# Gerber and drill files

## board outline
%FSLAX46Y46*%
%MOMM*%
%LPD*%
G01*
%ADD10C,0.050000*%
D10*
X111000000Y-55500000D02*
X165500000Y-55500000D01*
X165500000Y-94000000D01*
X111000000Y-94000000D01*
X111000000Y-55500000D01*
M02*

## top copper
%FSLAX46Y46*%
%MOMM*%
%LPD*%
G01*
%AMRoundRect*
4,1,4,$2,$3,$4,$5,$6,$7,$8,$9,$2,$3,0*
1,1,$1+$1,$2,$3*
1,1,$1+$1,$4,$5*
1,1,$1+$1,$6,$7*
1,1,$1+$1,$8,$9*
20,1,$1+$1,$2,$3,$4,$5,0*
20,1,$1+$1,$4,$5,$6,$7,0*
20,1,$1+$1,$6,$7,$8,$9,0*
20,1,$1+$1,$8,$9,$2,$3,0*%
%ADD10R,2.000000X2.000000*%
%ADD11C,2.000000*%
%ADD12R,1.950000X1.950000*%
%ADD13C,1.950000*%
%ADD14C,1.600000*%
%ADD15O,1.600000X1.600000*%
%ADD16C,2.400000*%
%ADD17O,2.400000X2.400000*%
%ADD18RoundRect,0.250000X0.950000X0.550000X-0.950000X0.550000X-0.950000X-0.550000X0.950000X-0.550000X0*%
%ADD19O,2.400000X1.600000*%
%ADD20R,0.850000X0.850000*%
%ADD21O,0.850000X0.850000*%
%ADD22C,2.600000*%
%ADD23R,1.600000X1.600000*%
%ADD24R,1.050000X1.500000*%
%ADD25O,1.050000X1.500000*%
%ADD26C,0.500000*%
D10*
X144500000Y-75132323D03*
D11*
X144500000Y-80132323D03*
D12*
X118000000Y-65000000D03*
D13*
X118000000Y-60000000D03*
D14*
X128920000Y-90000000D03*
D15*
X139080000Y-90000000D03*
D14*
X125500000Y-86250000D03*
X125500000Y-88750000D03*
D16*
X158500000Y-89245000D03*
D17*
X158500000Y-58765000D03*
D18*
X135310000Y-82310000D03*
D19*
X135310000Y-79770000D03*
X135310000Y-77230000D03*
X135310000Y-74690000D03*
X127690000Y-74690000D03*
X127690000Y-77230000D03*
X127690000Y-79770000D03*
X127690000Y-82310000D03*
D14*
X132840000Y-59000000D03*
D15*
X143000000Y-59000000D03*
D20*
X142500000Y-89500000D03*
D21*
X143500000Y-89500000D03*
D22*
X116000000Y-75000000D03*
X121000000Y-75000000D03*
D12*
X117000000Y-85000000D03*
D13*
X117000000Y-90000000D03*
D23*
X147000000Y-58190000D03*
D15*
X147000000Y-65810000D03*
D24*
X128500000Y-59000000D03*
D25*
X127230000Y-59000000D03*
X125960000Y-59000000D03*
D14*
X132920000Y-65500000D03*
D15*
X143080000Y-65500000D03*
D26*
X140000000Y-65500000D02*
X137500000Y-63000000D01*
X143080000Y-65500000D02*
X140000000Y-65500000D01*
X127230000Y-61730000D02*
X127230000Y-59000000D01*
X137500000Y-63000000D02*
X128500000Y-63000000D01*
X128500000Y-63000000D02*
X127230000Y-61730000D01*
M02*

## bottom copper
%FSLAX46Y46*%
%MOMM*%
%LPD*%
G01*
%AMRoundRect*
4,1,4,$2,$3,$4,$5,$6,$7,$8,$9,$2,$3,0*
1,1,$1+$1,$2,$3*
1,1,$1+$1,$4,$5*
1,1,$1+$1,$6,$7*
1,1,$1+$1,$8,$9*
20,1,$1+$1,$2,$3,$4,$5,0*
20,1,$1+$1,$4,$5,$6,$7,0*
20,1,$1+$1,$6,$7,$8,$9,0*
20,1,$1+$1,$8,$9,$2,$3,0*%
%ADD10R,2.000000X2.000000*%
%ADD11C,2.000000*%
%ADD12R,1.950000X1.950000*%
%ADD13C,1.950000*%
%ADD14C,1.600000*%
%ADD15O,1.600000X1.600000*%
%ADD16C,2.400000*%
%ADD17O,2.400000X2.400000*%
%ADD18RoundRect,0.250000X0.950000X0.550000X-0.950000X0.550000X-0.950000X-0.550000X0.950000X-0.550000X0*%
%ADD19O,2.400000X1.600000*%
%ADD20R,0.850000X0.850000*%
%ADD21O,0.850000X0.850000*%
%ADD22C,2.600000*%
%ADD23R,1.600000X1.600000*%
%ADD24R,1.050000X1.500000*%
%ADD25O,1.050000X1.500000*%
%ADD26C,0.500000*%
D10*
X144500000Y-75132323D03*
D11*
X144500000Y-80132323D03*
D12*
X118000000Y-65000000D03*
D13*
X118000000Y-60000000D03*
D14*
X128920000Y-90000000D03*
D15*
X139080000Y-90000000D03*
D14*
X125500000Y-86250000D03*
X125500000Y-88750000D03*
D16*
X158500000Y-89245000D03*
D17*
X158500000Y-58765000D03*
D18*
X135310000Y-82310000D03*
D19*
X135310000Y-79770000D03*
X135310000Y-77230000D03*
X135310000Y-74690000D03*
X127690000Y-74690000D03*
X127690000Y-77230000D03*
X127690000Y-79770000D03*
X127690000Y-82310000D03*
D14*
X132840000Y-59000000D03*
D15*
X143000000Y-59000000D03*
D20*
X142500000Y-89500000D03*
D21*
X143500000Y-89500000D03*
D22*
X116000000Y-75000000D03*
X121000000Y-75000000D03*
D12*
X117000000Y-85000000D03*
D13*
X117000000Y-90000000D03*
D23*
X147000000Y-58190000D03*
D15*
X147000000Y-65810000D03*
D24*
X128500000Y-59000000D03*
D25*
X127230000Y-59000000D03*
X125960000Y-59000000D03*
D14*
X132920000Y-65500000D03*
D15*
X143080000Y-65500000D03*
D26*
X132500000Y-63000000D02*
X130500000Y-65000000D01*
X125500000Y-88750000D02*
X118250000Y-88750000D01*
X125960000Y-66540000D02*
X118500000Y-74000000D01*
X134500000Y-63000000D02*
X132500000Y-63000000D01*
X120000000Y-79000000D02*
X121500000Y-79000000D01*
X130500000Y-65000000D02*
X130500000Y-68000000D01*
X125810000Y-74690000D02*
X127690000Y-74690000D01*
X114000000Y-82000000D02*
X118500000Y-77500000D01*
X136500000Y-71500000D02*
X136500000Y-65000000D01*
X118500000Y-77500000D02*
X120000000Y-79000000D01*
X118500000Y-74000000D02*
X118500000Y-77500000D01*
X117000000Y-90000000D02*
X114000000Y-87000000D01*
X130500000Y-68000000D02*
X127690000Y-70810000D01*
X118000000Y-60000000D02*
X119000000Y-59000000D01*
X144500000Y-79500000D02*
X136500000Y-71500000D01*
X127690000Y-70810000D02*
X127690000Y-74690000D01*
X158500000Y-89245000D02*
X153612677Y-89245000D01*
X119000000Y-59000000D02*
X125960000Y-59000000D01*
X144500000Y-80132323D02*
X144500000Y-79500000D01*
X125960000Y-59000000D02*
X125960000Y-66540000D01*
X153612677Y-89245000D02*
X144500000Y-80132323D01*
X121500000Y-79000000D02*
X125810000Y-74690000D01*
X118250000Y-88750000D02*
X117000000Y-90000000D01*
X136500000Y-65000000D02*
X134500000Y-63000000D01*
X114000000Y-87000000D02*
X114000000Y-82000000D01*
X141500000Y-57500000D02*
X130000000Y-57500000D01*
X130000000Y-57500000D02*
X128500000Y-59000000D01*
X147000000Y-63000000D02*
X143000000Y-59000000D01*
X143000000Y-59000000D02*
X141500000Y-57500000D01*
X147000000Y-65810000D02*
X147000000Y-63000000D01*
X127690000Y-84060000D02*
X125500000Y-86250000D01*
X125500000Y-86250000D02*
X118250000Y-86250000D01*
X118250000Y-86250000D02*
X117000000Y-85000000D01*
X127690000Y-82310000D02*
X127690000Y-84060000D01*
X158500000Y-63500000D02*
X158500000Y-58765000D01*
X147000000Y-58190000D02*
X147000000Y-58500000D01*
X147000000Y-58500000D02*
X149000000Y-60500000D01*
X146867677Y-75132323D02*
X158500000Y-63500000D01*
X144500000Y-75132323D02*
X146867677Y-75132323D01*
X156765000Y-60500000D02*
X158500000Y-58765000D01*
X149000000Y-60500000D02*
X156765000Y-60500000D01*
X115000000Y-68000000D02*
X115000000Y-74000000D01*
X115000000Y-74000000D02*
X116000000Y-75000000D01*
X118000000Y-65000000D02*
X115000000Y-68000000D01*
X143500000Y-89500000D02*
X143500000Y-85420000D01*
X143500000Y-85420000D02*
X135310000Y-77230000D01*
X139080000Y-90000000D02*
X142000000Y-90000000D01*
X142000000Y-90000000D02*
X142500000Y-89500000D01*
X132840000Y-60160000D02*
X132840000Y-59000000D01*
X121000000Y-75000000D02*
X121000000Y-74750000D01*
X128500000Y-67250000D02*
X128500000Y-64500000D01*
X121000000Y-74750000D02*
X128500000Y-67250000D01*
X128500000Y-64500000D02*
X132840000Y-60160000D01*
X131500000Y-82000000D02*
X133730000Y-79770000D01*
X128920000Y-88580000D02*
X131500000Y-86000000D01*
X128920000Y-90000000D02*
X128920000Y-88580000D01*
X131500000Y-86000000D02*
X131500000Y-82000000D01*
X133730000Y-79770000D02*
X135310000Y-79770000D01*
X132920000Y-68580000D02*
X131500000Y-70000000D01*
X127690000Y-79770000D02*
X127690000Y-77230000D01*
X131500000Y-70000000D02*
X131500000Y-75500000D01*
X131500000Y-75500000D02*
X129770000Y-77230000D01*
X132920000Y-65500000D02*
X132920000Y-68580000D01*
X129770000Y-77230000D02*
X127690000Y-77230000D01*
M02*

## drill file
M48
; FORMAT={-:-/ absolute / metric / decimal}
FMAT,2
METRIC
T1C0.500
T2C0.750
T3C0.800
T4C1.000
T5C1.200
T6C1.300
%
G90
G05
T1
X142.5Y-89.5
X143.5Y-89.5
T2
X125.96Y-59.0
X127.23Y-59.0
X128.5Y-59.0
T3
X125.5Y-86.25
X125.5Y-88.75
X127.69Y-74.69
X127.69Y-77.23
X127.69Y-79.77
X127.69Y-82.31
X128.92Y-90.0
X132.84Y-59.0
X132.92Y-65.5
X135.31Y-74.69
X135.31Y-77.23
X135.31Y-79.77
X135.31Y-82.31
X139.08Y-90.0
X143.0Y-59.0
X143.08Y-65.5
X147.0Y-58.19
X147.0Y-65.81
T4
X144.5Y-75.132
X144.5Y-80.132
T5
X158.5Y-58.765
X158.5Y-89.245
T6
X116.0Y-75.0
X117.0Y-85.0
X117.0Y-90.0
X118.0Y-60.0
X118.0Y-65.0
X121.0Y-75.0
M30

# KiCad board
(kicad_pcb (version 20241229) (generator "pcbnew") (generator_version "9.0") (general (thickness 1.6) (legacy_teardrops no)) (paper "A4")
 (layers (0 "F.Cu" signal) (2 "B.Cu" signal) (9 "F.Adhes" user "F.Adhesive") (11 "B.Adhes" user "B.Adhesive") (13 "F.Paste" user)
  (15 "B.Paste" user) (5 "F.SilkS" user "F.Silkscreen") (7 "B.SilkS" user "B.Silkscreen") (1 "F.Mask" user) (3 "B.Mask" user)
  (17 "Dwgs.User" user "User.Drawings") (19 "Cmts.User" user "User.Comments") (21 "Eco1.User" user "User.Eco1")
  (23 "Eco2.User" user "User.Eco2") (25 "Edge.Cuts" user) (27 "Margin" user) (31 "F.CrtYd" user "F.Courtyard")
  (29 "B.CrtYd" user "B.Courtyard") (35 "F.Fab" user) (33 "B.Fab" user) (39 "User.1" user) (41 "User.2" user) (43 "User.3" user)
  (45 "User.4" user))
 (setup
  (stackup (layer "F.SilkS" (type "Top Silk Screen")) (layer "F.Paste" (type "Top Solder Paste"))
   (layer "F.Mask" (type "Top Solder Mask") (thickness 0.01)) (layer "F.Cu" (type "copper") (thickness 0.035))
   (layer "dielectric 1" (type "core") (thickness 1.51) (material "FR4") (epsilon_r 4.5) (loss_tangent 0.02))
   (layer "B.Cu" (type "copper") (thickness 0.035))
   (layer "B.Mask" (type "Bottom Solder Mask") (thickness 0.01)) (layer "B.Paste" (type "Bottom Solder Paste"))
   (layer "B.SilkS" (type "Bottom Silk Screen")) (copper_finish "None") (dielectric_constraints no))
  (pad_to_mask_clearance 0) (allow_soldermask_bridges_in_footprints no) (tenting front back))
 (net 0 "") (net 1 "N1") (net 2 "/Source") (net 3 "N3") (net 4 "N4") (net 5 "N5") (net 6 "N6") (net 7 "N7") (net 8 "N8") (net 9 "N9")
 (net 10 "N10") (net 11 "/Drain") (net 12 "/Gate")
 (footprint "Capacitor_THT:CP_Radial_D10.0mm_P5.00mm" (layer "F.Cu") (at 144.5 75.132323 -90)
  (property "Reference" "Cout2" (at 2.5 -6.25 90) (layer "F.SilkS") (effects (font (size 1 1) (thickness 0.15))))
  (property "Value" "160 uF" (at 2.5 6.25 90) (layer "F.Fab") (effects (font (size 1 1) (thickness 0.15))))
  (pad "1" thru_hole rect (at 0 0 270) (size 2 2) (drill 1) (layers "*.Cu" "*.Mask") (remove_unused_layers no) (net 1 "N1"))
  (pad "2" thru_hole circle (at 5 0 270) (size 2 2) (drill 1) (layers "*.Cu" "*.Mask") (remove_unused_layers no) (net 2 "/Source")))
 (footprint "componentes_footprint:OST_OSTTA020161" (layer "F.Cu") (at 118 62.5 90)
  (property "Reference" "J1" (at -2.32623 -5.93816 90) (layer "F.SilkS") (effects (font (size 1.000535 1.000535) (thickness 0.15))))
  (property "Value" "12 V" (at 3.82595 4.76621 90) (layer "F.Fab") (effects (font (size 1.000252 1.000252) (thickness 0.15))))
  (pad "1" thru_hole rect (at -2.5 0 90) (size 1.95 1.95) (drill 1.3) (layers "*.Cu" "*.Mask") (remove_unused_layers no) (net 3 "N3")
   (solder_mask_margin 0.102))
  (pad "2" thru_hole circle (at 2.5 0 90) (size 1.95 1.95) (drill 1.3) (layers "*.Cu" "*.Mask") (remove_unused_layers no) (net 2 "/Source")
   (solder_mask_margin 0.102)))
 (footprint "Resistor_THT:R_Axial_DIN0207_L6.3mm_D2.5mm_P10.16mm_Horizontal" (layer "F.Cu") (at 128.92 90)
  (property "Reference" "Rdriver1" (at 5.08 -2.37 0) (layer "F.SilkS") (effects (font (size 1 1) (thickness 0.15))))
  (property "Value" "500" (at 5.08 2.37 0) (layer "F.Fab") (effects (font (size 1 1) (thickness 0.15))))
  (pad "1" thru_hole circle (at 0 0) (size 1.6 1.6) (drill 0.8) (layers "*.Cu" "*.Mask") (remove_unused_layers no) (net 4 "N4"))
  (pad "2" thru_hole oval (at 10.16 0) (size 1.6 1.6) (drill 0.8) (layers "*.Cu" "*.Mask") (remove_unused_layers no) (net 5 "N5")))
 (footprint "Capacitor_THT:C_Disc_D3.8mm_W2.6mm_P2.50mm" (layer "F.Cu") (at 125.5 86.25 -90)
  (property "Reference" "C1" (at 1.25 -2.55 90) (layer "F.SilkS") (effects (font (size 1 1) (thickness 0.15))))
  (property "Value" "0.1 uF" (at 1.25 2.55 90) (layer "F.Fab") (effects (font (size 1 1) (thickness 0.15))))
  (pad "1" thru_hole circle (at 0 0 270) (size 1.6 1.6) (drill 0.8) (layers "*.Cu" "*.Mask") (remove_unused_layers no) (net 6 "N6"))
  (pad "2" thru_hole circle (at 2.5 0 270) (size 1.6 1.6) (drill 0.8) (layers "*.Cu" "*.Mask") (remove_unused_layers no) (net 2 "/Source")))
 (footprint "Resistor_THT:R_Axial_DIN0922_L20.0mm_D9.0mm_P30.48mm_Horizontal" (layer "F.Cu") (at 158.5 89.245 90)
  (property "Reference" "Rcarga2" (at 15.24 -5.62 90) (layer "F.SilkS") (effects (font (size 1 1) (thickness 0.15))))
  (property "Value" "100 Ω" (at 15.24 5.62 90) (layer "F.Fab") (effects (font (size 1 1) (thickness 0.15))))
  (pad "1" thru_hole circle (at 0 0 90) (size 2.4 2.4) (drill 1.2) (layers "*.Cu" "*.Mask") (remove_unused_layers no) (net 2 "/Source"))
  (pad "2" thru_hole oval (at 30.48 0 90) (size 2.4 2.4) (drill 1.2) (layers "*.Cu" "*.Mask") (remove_unused_layers no) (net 1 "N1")))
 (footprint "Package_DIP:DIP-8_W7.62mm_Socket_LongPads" (layer "F.Cu") (at 135.31 82.31 180)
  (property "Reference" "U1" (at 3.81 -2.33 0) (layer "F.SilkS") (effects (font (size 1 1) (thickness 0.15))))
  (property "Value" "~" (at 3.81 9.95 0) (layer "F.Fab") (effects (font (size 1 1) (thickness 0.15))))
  (pad "1" thru_hole roundrect (at 0 0 180) (size 2.4 1.6) (drill 0.8) (layers "*.Cu" "*.Mask") (remove_unused_layers no)
   (roundrect_rratio 0.15625) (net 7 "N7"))
  (pad "2" thru_hole oval (at 0 2.54 180) (size 2.4 1.6) (drill 0.8) (layers "*.Cu" "*.Mask") (remove_unused_layers no) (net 4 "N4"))
  (pad "3" thru_hole oval (at 0 5.08 180) (size 2.4 1.6) (drill 0.8) (layers "*.Cu" "*.Mask") (remove_unused_layers no) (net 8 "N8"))
  (pad "4" thru_hole oval (at 0 7.62 180) (size 2.4 1.6) (drill 0.8) (layers "*.Cu" "*.Mask") (remove_unused_layers no))
  (pad "5" thru_hole oval (at 7.62 7.62 180) (size 2.4 1.6) (drill 0.8) (layers "*.Cu" "*.Mask") (remove_unused_layers no) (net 2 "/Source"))
  (pad "6" thru_hole oval (at 7.62 5.08 180) (size 2.4 1.6) (drill 0.8) (layers "*.Cu" "*.Mask") (remove_unused_layers no) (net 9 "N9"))
  (pad "7" thru_hole oval (at 7.62 2.54 180) (size 2.4 1.6) (drill 0.8) (layers "*.Cu" "*.Mask") (remove_unused_layers no) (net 9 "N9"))
  (pad "8" thru_hole oval (at 7.62 0 180) (size 2.4 1.6) (drill 0.8) (layers "*.Cu" "*.Mask") (remove_unused_layers no) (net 6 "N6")))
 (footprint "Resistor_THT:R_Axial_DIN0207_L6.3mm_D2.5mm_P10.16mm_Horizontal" (layer "F.Cu") (at 132.84 59)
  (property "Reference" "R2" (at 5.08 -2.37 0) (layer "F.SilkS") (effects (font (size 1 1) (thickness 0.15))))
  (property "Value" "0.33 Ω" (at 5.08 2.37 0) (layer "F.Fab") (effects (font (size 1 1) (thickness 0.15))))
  (pad "1" thru_hole circle (at 0 0) (size 1.6 1.6) (drill 0.8) (layers "*.Cu" "*.Mask") (remove_unused_layers no) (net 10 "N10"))
  (pad "2" thru_hole oval (at 10.16 0) (size 1.6 1.6) (drill 0.8) (layers "*.Cu" "*.Mask") (remove_unused_layers no) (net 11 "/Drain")))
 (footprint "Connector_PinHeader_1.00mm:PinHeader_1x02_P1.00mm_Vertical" (layer "F.Cu") (at 142.5 89.5 90)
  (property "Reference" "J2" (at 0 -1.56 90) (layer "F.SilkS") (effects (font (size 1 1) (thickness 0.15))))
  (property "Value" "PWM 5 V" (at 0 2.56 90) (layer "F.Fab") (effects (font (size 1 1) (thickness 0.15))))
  (pad "1" thru_hole rect (at 0 0 90) (size 0.85 0.85) (drill 0.5) (layers "*.Cu" "*.Mask") (remove_unused_layers no) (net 5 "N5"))
  (pad "2" thru_hole oval (at 0 1 90) (size 0.85 0.85) (drill 0.5) (layers "*.Cu" "*.Mask") (remove_unused_layers no) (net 8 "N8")))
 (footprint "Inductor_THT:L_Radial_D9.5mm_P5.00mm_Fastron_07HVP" (layer "F.Cu") (at 116 75)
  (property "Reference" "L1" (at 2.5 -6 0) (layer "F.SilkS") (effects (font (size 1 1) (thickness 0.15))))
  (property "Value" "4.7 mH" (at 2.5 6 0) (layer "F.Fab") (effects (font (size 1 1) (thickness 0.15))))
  (pad "1" thru_hole circle (at 0 0) (size 2.6 2.6) (drill 1.3) (layers "*.Cu" "*.Mask") (remove_unused_layers no) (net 3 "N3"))
  (pad "2" thru_hole circle (at 5 0) (size 2.6 2.6) (drill 1.3) (layers "*.Cu" "*.Mask") (remove_unused_layers no) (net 10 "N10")))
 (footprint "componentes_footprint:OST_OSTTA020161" (layer "F.Cu") (at 117 87.5 -90)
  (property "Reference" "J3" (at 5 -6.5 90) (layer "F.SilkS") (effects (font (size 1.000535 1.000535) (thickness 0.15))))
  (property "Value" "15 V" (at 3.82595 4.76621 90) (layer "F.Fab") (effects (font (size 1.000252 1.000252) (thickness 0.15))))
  (pad "1" thru_hole rect (at -2.5 0 270) (size 1.95 1.95) (drill 1.3) (layers "*.Cu" "*.Mask") (remove_unused_layers no) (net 6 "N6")
   (solder_mask_margin 0.102))
  (pad "2" thru_hole circle (at 2.5 0 270) (size 1.95 1.95) (drill 1.3) (layers "*.Cu" "*.Mask") (remove_unused_layers no) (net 2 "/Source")
   (solder_mask_margin 0.102)))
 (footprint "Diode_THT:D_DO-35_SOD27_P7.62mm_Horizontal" (layer "F.Cu") (at 147 58.19 -90)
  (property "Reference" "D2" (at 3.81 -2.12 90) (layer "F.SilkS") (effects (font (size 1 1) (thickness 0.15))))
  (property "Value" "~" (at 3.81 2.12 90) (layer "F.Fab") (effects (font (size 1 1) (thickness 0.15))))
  (pad "1" thru_hole rect (at 0 0 270) (size 1.6 1.6) (drill 0.8) (layers "*.Cu" "*.Mask") (remove_unused_layers no) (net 1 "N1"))
  (pad "2" thru_hole oval (at 7.62 0 270) (size 1.6 1.6) (drill 0.8) (layers "*.Cu" "*.Mask") (remove_unused_layers no) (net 11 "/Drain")))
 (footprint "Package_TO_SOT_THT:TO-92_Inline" (layer "F.Cu") (at 128.5 59 180)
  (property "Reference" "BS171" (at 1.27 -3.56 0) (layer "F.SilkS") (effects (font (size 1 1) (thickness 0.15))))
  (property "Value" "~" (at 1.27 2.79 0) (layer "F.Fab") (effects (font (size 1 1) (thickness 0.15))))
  (pad "1" thru_hole rect (at 0 0 180) (size 1.05 1.5) (drill 0.75) (layers "*.Cu" "*.Mask") (remove_unused_layers no) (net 11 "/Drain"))
  (pad "2" thru_hole oval (at 1.27 0 180) (size 1.05 1.5) (drill 0.75) (layers "*.Cu" "*.Mask") (remove_unused_layers no) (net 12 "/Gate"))
  (pad "3" thru_hole oval (at 2.54 0 180) (size 1.05 1.5) (drill 0.75) (layers "*.Cu" "*.Mask") (remove_unused_layers no) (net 2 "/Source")))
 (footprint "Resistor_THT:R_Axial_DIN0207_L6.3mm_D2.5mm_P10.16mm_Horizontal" (layer "F.Cu") (at 132.92 65.5)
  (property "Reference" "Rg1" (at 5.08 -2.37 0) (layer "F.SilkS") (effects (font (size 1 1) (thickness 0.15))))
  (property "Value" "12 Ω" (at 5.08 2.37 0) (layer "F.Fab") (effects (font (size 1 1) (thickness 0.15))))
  (pad "1" thru_hole circle (at 0 0) (size 1.6 1.6) (drill 0.8) (layers "*.Cu" "*.Mask") (remove_unused_layers no) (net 9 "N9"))
  (pad "2" thru_hole oval (at 10.16 0) (size 1.6 1.6) (drill 0.8) (layers "*.Cu" "*.Mask") (remove_unused_layers no) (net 12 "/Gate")))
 (gr_rect (start 111 55.5) (end 165.5 94) (stroke (width 0.05) (type default)) (fill no) (layer "Edge.Cuts"))
 (segment (start 132.5 63) (end 130.5 65) (width 0.5) (layer "B.Cu") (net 2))
 (segment (start 125.5 88.75) (end 118.25 88.75) (width 0.5) (layer "B.Cu") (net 2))
 (segment (start 125.96 66.54) (end 118.5 74) (width 0.5) (layer "B.Cu") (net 2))
 (segment (start 134.5 63) (end 132.5 63) (width 0.5) (layer "B.Cu") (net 2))
 (segment (start 120 79) (end 121.5 79) (width 0.5) (layer "B.Cu") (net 2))
 (segment (start 130.5 65) (end 130.5 68) (width 0.5) (layer "B.Cu") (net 2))
 (segment (start 125.81 74.69) (end 127.69 74.69) (width 0.5) (layer "B.Cu") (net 2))
 (segment (start 114 82) (end 118.5 77.5) (width 0.5) (layer "B.Cu") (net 2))
 (segment (start 136.5 71.5) (end 136.5 65) (width 0.5) (layer "B.Cu") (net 2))
 (segment (start 118.5 77.5) (end 120 79) (width 0.5) (layer "B.Cu") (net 2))
 (segment (start 118.5 74) (end 118.5 77.5) (width 0.5) (layer "B.Cu") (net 2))
 (segment (start 117 90) (end 114 87) (width 0.5) (layer "B.Cu") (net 2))
 (segment (start 130.5 68) (end 127.69 70.81) (width 0.5) (layer "B.Cu") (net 2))
 (segment (start 118 60) (end 119 59) (width 0.5) (layer "B.Cu") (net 2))
 (segment (start 144.5 79.5) (end 136.5 71.5) (width 0.5) (layer "B.Cu") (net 2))
 (segment (start 127.69 70.81) (end 127.69 74.69) (width 0.5) (layer "B.Cu") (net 2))
 (segment (start 158.5 89.245) (end 153.612677 89.245) (width 0.5) (layer "B.Cu") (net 2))
 (segment (start 119 59) (end 125.96 59) (width 0.5) (layer "B.Cu") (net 2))
 (segment (start 144.5 80.132323) (end 144.5 79.5) (width 0.5) (layer "B.Cu") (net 2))
 (segment (start 125.96 59) (end 125.96 66.54) (width 0.5) (layer "B.Cu") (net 2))
 (segment (start 153.612677 89.245) (end 144.5 80.132323) (width 0.5) (layer "B.Cu") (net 2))
 (segment (start 121.5 79) (end 125.81 74.69) (width 0.5) (layer "B.Cu") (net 2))
 (segment (start 118.25 88.75) (end 117 90) (width 0.5) (layer "B.Cu") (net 2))
 (segment (start 136.5 65) (end 134.5 63) (width 0.5) (layer "B.Cu") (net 2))
 (segment (start 114 87) (end 114 82) (width 0.5) (layer "B.Cu") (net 2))
 (segment (start 141.5 57.5) (end 130 57.5) (width 0.5) (layer "B.Cu") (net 11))
 (segment (start 130 57.5) (end 128.5 59) (width 0.5) (layer "B.Cu") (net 11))
 (segment (start 147 63) (end 143 59) (width 0.5) (layer "B.Cu") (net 11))
 (segment (start 143 59) (end 141.5 57.5) (width 0.5) (layer "B.Cu") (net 11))
 (segment (start 147 65.81) (end 147 63) (width 0.5) (layer "B.Cu") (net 11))
 (segment (start 140 65.5) (end 137.5 63) (width 0.5) (layer "F.Cu") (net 12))
 (segment (start 143.08 65.5) (end 140 65.5) (width 0.5) (layer "F.Cu") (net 12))
 (segment (start 127.23 61.73) (end 127.23 59) (width 0.5) (layer "F.Cu") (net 12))
 (segment (start 137.5 63) (end 128.5 63) (width 0.5) (layer "F.Cu") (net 12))
 (segment (start 128.5 63) (end 127.23 61.73) (width 0.5) (layer "F.Cu") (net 12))
 (segment (start 127.69 84.06) (end 125.5 86.25) (width 0.5) (layer "B.Cu") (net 6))
 (segment (start 125.5 86.25) (end 118.25 86.25) (width 0.5) (layer "B.Cu") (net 6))
 (segment (start 118.25 86.25) (end 117 85) (width 0.5) (layer "B.Cu") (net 6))
 (segment (start 127.69 82.31) (end 127.69 84.06) (width 0.5) (layer "B.Cu") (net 6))
 (segment (start 158.5 63.5) (end 158.5 58.765) (width 0.5) (layer "B.Cu") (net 1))
 (segment (start 147 58.19) (end 147 58.5) (width 0.5) (layer "B.Cu") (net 1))
 (segment (start 147 58.5) (end 149 60.5) (width 0.5) (layer "B.Cu") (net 1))
 (segment (start 146.867677 75.132323) (end 158.5 63.5) (width 0.5) (layer "B.Cu") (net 1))
 (segment (start 144.5 75.132323) (end 146.867677 75.132323) (width 0.5) (layer "B.Cu") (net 1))
 (segment (start 156.765 60.5) (end 158.5 58.765) (width 0.5) (layer "B.Cu") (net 1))
 (segment (start 149 60.5) (end 156.765 60.5) (width 0.5) (layer "B.Cu") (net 1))
 (segment (start 115 68) (end 115 74) (width 0.5) (layer "B.Cu") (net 3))
 (segment (start 115 74) (end 116 75) (width 0.5) (layer "B.Cu") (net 3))
 (segment (start 118 65) (end 115 68) (width 0.5) (layer "B.Cu") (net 3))
 (segment (start 143.5 89.5) (end 143.5 85.42) (width 0.5) (layer "B.Cu") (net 8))
 (segment (start 143.5 85.42) (end 135.31 77.23) (width 0.5) (layer "B.Cu") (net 8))
 (segment (start 139.08 90) (end 142 90) (width 0.5) (layer "B.Cu") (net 5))
 (segment (start 142 90) (end 142.5 89.5) (width 0.5) (layer "B.Cu") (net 5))
 (segment (start 132.84 60.16) (end 132.84 59) (width 0.5) (layer "B.Cu") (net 10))
 (segment (start 121 75) (end 121 74.75) (width 0.5) (layer "B.Cu") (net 10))
 (segment (start 128.5 67.25) (end 128.5 64.5) (width 0.5) (layer "B.Cu") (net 10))
 (segment (start 121 74.75) (end 128.5 67.25) (width 0.5) (layer "B.Cu") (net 10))
 (segment (start 128.5 64.5) (end 132.84 60.16) (width 0.5) (layer "B.Cu") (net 10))
 (segment (start 131.5 82) (end 133.73 79.77) (width 0.5) (layer "B.Cu") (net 4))
 (segment (start 128.92 88.58) (end 131.5 86) (width 0.5) (layer "B.Cu") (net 4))
 (segment (start 128.92 90) (end 128.92 88.58) (width 0.5) (layer "B.Cu") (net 4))
 (segment (start 131.5 86) (end 131.5 82) (width 0.5) (layer "B.Cu") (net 4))
 (segment (start 133.73 79.77) (end 135.31 79.77) (width 0.5) (layer "B.Cu") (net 4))
 (segment (start 132.92 68.58) (end 131.5 70) (width 0.5) (layer "B.Cu") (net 9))
 (segment (start 127.69 79.77) (end 127.69 77.23) (width 0.5) (layer "B.Cu") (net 9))
 (segment (start 131.5 70) (end 131.5 75.5) (width 0.5) (layer "B.Cu") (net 9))
 (segment (start 131.5 75.5) (end 129.77 77.23) (width 0.5) (layer "B.Cu") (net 9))
 (segment (start 132.92 65.5) (end 132.92 68.58) (width 0.5) (layer "B.Cu") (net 9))
 (segment (start 129.77 77.23) (end 127.69 77.23) (width 0.5) (layer "B.Cu") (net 9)))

